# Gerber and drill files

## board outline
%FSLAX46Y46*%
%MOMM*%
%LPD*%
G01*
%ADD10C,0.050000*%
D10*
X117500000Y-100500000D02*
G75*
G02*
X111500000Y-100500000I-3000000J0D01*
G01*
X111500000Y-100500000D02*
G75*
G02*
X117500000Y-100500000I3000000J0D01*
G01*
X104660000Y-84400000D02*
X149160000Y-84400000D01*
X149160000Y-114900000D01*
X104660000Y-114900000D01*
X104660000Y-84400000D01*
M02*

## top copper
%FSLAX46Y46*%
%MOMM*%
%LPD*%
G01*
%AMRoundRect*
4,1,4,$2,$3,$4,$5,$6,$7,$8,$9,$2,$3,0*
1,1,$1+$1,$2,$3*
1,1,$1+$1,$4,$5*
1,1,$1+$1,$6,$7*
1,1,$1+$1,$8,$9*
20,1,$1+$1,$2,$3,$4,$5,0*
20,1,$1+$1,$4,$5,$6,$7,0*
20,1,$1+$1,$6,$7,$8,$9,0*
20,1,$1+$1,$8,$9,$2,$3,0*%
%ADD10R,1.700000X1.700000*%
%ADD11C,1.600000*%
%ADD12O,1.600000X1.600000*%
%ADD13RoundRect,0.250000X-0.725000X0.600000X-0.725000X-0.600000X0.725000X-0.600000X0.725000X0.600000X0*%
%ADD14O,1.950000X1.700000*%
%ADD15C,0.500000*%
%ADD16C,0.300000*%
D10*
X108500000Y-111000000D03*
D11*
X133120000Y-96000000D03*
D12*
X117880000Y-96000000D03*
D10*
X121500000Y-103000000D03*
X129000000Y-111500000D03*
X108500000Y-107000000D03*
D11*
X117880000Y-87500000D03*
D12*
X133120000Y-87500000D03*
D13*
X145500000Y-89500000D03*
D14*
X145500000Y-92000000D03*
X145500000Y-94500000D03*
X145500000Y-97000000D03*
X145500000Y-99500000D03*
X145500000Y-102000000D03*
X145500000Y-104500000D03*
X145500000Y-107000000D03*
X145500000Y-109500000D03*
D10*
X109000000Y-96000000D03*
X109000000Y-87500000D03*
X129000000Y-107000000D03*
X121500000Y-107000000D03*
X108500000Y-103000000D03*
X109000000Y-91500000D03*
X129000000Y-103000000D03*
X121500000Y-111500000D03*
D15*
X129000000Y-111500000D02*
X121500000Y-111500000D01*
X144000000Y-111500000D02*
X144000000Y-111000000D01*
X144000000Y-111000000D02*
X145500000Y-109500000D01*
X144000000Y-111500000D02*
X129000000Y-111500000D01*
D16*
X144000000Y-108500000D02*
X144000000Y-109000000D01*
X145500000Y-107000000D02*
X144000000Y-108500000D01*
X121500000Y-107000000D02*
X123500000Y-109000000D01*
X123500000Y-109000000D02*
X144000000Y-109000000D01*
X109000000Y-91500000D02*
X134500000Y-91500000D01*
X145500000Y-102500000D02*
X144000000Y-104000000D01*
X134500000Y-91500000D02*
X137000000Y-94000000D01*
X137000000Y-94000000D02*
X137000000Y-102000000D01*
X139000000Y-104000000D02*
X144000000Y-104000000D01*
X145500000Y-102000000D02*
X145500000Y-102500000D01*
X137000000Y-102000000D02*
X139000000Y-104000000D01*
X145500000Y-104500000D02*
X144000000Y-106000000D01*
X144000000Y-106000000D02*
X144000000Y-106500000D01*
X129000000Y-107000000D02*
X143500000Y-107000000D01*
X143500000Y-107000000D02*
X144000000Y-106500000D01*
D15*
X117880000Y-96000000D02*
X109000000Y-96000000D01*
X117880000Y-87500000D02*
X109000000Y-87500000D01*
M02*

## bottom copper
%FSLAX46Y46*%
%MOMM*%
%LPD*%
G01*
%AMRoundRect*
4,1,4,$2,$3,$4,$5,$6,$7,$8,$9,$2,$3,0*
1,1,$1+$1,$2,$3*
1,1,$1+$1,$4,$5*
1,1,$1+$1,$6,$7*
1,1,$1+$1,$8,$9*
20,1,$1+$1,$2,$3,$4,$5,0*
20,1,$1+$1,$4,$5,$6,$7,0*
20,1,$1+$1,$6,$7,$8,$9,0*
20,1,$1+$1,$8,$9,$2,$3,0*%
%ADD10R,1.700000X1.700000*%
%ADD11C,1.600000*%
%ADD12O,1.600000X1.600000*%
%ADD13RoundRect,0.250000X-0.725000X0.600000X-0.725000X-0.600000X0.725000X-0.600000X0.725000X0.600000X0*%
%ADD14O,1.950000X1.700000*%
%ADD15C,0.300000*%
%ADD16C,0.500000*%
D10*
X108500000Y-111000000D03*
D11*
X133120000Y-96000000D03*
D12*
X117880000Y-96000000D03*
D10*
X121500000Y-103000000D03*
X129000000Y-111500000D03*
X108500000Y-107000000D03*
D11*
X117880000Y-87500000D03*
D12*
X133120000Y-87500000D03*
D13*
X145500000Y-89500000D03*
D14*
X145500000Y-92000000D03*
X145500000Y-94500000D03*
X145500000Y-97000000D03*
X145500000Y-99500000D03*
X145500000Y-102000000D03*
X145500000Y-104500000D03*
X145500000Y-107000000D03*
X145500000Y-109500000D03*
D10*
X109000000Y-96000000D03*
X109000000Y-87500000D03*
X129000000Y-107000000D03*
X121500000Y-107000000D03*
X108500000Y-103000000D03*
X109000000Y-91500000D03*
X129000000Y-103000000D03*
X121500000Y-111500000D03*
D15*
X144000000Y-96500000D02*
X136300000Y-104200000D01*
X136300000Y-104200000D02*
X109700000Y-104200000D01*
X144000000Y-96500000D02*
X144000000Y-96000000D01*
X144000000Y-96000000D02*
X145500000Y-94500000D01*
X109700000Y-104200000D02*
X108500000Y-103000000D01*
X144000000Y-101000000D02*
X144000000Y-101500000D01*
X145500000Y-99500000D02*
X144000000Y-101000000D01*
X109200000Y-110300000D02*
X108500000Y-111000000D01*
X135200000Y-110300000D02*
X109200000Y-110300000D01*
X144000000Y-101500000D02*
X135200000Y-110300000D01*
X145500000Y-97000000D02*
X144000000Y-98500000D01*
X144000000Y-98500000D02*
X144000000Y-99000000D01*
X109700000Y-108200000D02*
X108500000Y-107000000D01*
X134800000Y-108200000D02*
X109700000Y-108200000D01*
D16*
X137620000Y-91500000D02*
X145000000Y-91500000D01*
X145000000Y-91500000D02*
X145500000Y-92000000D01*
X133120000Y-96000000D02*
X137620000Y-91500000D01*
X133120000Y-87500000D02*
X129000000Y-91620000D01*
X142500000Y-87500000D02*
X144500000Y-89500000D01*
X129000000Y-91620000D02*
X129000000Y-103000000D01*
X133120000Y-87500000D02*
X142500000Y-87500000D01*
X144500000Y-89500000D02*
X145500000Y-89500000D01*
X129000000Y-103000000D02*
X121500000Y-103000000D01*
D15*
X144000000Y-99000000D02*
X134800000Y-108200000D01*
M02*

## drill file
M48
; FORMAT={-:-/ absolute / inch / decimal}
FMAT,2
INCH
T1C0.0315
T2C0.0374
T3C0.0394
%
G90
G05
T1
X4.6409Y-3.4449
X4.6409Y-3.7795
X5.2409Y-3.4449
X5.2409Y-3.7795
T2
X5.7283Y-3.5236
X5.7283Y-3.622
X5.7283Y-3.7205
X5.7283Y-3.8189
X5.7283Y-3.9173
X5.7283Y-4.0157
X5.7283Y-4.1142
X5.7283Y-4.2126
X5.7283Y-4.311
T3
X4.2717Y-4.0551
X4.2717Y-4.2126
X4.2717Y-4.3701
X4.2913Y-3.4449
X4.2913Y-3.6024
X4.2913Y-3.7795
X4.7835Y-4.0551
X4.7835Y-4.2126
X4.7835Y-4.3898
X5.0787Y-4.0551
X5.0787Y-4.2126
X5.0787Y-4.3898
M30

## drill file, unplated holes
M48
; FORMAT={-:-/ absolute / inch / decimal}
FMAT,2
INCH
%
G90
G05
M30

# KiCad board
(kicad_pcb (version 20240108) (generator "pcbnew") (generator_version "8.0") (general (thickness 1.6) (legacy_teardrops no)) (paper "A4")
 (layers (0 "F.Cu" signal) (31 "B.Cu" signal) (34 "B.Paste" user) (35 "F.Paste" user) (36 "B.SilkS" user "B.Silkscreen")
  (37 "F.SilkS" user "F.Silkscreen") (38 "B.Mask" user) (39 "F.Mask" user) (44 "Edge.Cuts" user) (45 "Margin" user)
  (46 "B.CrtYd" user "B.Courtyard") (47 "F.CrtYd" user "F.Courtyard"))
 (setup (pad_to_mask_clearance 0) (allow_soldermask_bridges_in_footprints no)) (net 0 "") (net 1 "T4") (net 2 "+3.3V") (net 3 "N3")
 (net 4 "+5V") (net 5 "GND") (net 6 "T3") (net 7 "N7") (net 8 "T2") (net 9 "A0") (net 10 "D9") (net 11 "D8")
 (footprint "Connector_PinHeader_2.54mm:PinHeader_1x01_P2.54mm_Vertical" (layer "F.Cu") (at 108.5 111 -90)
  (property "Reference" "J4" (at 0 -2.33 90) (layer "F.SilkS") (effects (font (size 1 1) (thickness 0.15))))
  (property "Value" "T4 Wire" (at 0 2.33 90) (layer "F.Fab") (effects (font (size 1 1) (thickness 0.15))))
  (pad "1" thru_hole rect (at 0 0 270) (size 1.7 1.7) (drill 1) (layers "*.Cu" "*.Mask") (remove_unused_layers no) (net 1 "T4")))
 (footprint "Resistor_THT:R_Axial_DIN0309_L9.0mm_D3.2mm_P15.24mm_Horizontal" (layer "F.Cu") (at 133.12 96 180)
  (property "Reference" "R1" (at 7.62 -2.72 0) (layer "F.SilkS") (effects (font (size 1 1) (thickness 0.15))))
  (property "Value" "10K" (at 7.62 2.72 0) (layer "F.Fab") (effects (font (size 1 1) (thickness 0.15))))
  (pad "1" thru_hole circle (at 0 0 180) (size 1.6 1.6) (drill 0.8) (layers "*.Cu" "*.Mask") (remove_unused_layers no) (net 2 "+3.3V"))
  (pad "2" thru_hole oval (at 15.24 0 180) (size 1.6 1.6) (drill 0.8) (layers "*.Cu" "*.Mask") (remove_unused_layers no) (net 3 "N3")))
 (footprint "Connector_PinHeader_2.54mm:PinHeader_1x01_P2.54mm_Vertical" (layer "F.Cu") (at 121.5 103 -90)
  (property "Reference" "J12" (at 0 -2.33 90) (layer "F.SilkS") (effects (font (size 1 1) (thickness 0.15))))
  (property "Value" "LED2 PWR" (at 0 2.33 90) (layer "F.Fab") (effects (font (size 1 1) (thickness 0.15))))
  (pad "1" thru_hole rect (at 0 0 270) (size 1.7 1.7) (drill 1) (layers "*.Cu" "*.Mask") (remove_unused_layers no) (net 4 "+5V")))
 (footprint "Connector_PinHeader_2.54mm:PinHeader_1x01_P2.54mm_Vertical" (layer "F.Cu") (at 129 111.5 -90)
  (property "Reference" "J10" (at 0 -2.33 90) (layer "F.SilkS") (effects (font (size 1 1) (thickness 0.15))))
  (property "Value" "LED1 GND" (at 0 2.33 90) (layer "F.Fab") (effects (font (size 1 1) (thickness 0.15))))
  (pad "1" thru_hole rect (at 0 0 270) (size 1.7 1.7) (drill 1) (layers "*.Cu" "*.Mask") (remove_unused_layers no) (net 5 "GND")))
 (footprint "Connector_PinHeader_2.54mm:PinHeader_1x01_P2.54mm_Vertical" (layer "F.Cu") (at 108.5 107 -90)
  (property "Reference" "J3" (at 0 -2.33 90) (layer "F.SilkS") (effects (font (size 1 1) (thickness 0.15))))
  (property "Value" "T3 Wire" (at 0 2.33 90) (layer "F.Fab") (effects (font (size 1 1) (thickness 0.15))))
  (pad "1" thru_hole rect (at 0 0 270) (size 1.7 1.7) (drill 1) (layers "*.Cu" "*.Mask") (remove_unused_layers no) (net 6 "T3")))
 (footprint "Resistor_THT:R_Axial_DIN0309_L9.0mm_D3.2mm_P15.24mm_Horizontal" (layer "F.Cu") (at 117.88 87.5)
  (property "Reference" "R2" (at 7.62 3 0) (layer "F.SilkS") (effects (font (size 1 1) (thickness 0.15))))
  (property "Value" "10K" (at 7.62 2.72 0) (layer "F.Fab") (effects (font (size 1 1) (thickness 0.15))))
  (pad "1" thru_hole circle (at 0 0) (size 1.6 1.6) (drill 0.8) (layers "*.Cu" "*.Mask") (remove_unused_layers no) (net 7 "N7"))
  (pad "2" thru_hole oval (at 15.24 0) (size 1.6 1.6) (drill 0.8) (layers "*.Cu" "*.Mask") (remove_unused_layers no) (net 4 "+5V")))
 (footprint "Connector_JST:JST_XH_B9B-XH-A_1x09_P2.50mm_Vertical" (layer "F.Cu") (at 145.5 89.5 -90)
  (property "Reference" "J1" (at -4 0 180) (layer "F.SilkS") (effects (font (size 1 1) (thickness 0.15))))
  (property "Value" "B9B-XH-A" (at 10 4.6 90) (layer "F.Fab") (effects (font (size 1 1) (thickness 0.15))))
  (pad "1" thru_hole roundrect (at 0 0 270) (size 1.7 1.95) (drill 0.95) (layers "*.Cu" "*.Mask") (remove_unused_layers no)
   (roundrect_rratio 0.147059) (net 4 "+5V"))
  (pad "2" thru_hole oval (at 2.5 0 270) (size 1.7 1.95) (drill 0.95) (layers "*.Cu" "*.Mask") (remove_unused_layers no) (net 2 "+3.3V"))
  (pad "3" thru_hole oval (at 5 0 270) (size 1.7 1.95) (drill 0.95) (layers "*.Cu" "*.Mask") (remove_unused_layers no) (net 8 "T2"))
  (pad "4" thru_hole oval (at 7.5 0 270) (size 1.7 1.95) (drill 0.95) (layers "*.Cu" "*.Mask") (remove_unused_layers no) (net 6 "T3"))
  (pad "5" thru_hole oval (at 10 0 270) (size 1.7 1.95) (drill 0.95) (layers "*.Cu" "*.Mask") (remove_unused_layers no) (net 1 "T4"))
  (pad "6" thru_hole oval (at 12.5 0 270) (size 1.7 1.95) (drill 0.95) (layers "*.Cu" "*.Mask") (remove_unused_layers no) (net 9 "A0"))
  (pad "7" thru_hole oval (at 15 0 270) (size 1.7 1.95) (drill 0.95) (layers "*.Cu" "*.Mask") (remove_unused_layers no) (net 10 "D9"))
  (pad "8" thru_hole oval (at 17.5 0 270) (size 1.7 1.95) (drill 0.95) (layers "*.Cu" "*.Mask") (remove_unused_layers no) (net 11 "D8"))
  (pad "9" thru_hole oval (at 20 0 270) (size 1.7 1.95) (drill 0.95) (layers "*.Cu" "*.Mask") (remove_unused_layers no) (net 5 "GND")))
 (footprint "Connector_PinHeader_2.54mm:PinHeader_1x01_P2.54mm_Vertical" (layer "F.Cu") (at 109 96 -90)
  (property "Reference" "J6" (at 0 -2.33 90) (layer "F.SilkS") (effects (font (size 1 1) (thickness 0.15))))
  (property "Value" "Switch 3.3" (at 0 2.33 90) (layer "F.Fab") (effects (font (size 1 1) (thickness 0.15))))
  (pad "1" thru_hole rect (at 0 0 270) (size 1.7 1.7) (drill 1) (layers "*.Cu" "*.Mask") (remove_unused_layers no) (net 3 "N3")))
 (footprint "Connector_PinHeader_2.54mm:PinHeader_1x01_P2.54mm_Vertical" (layer "F.Cu") (at 109 87.5 -90)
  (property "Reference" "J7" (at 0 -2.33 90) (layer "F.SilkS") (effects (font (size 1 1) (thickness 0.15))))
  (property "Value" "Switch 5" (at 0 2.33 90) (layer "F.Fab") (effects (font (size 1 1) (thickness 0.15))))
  (pad "1" thru_hole rect (at 0 0 270) (size 1.7 1.7) (drill 1) (layers "*.Cu" "*.Mask") (remove_unused_layers no) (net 7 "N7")))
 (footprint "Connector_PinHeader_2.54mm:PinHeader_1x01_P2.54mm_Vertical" (layer "F.Cu") (at 129 107 -90)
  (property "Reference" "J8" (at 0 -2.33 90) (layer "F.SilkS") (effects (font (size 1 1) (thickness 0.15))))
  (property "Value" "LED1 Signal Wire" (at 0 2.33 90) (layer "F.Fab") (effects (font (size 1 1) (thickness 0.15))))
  (pad "1" thru_hole rect (at 0 0 270) (size 1.7 1.7) (drill 1) (layers "*.Cu" "*.Mask") (remove_unused_layers no) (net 10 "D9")))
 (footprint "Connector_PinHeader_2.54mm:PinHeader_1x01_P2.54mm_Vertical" (layer "F.Cu") (at 121.5 107 -90)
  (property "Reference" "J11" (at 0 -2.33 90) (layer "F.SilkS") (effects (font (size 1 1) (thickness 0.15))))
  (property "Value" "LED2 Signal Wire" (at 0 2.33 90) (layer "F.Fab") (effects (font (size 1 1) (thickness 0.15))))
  (pad "1" thru_hole rect (at 0 0 270) (size 1.7 1.7) (drill 1) (layers "*.Cu" "*.Mask") (remove_unused_layers no) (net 11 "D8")))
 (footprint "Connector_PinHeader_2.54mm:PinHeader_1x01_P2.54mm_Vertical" (layer "F.Cu") (at 108.5 103 -90)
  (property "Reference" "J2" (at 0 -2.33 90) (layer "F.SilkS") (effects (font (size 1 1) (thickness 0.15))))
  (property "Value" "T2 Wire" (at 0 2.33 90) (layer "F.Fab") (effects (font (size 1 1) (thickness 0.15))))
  (pad "1" thru_hole rect (at 0 0 270) (size 1.7 1.7) (drill 1) (layers "*.Cu" "*.Mask") (remove_unused_layers no) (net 8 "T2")))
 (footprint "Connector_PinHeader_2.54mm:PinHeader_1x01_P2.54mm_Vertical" (layer "F.Cu") (at 109 91.5 -90)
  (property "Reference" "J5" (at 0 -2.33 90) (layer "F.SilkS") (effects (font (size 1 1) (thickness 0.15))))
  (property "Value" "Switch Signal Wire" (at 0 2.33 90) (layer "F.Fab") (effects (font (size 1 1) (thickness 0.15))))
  (pad "1" thru_hole rect (at 0 0 270) (size 1.7 1.7) (drill 1) (layers "*.Cu" "*.Mask") (remove_unused_layers no) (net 9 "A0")))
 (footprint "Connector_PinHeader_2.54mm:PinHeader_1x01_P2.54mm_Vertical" (layer "F.Cu") (at 129 103 -90)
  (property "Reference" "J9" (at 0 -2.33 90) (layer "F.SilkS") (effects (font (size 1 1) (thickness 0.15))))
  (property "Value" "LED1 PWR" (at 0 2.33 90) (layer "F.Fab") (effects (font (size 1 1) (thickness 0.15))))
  (pad "1" thru_hole rect (at 0 0 270) (size 1.7 1.7) (drill 1) (layers "*.Cu" "*.Mask") (remove_unused_layers no) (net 4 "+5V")))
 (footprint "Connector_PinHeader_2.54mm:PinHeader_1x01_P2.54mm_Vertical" (layer "F.Cu") (at 121.5 111.5 -90)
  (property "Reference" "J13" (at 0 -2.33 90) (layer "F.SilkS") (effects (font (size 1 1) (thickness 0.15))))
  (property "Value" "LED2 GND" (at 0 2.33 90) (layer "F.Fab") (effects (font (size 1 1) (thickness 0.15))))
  (pad "1" thru_hole rect (at 0 0 270) (size 1.7 1.7) (drill 1) (layers "*.Cu" "*.Mask") (remove_unused_layers no) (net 5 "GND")))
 (gr_circle (center 114.5 100.5) (end 117.5 100.5) (stroke (width 0.05) (type default)) (fill none) (layer "Edge.Cuts"))
 (gr_rect (start 104.66 84.4) (end 149.16 114.9) (stroke (width 0.05) (type default)) (fill none) (layer "Edge.Cuts"))
 (segment (start 144 96.5) (end 136.3 104.2) (width 0.3) (layer "B.Cu") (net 8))
 (segment (start 136.3 104.2) (end 109.7 104.2) (width 0.3) (layer "B.Cu") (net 8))
 (segment (start 144 96.5) (end 144 96) (width 0.3) (layer "B.Cu") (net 8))
 (segment (start 144 96) (end 145.5 94.5) (width 0.3) (layer "B.Cu") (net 8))
 (segment (start 109.7 104.2) (end 108.5 103) (width 0.3) (layer "B.Cu") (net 8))
 (segment (start 129 111.5) (end 121.5 111.5) (width 0.5) (layer "F.Cu") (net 5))
 (segment (start 144 111.5) (end 144 111) (width 0.5) (layer "F.Cu") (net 5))
 (segment (start 144 111) (end 145.5 109.5) (width 0.5) (layer "F.Cu") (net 5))
 (segment (start 144 111.5) (end 129 111.5) (width 0.5) (layer "F.Cu") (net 5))
 (segment (start 144 108.5) (end 144 109) (width 0.3) (layer "F.Cu") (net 11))
 (segment (start 145.5 107) (end 144 108.5) (width 0.3) (layer "F.Cu") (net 11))
 (segment (start 121.5 107) (end 123.5 109) (width 0.3) (layer "F.Cu") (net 11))
 (segment (start 123.5 109) (end 144 109) (width 0.3) (layer "F.Cu") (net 11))
 (segment (start 144 101) (end 144 101.5) (width 0.3) (layer "B.Cu") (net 1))
 (segment (start 145.5 99.5) (end 144 101) (width 0.3) (layer "B.Cu") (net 1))
 (segment (start 109.2 110.3) (end 108.5 111) (width 0.3) (layer "B.Cu") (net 1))
 (segment (start 135.2 110.3) (end 109.2 110.3) (width 0.3) (layer "B.Cu") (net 1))
 (segment (start 144 101.5) (end 135.2 110.3) (width 0.3) (layer "B.Cu") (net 1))
 (segment (start 109 91.5) (end 134.5 91.5) (width 0.3) (layer "F.Cu") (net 9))
 (segment (start 145.5 102.5) (end 144 104) (width 0.3) (layer "F.Cu") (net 9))
 (segment (start 134.5 91.5) (end 137 94) (width 0.3) (layer "F.Cu") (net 9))
 (segment (start 137 94) (end 137 102) (width 0.3) (layer "F.Cu") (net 9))
 (segment (start 139 104) (end 144 104) (width 0.3) (layer "F.Cu") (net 9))
 (segment (start 145.5 102) (end 145.5 102.5) (width 0.3) (layer "F.Cu") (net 9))
 (segment (start 137 102) (end 139 104) (width 0.3) (layer "F.Cu") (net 9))
 (segment (start 145.5 97) (end 144 98.5) (width 0.3) (layer "B.Cu") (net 6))
 (segment (start 144 99) (end 134.8 108.2) (width 0.3) (layer "B.Cu") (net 6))
 (segment (start 144 98.5) (end 144 99) (width 0.3) (layer "B.Cu") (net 6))
 (segment (start 109.7 108.2) (end 108.5 107) (width 0.3) (layer "B.Cu") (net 6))
 (segment (start 134.8 108.2) (end 109.7 108.2) (width 0.3) (layer "B.Cu") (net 6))
 (segment (start 137.62 91.5) (end 145 91.5) (width 0.5) (layer "B.Cu") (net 2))
 (segment (start 145 91.5) (end 145.5 92) (width 0.5) (layer "B.Cu") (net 2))
 (segment (start 133.12 96) (end 137.62 91.5) (width 0.5) (layer "B.Cu") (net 2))
 (segment (start 145.5 104.5) (end 144 106) (width 0.3) (layer "F.Cu") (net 10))
 (segment (start 144 106) (end 144 106.5) (width 0.3) (layer "F.Cu") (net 10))
 (segment (start 129 107) (end 143.5 107) (width 0.3) (layer "F.Cu") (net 10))
 (segment (start 143.5 107) (end 144 106.5) (width 0.3) (layer "F.Cu") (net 10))
 (segment (start 117.88 96) (end 109 96) (width 0.5) (layer "F.Cu") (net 3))
 (segment (start 117.88 87.5) (end 109 87.5) (width 0.5) (layer "F.Cu") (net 7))
 (segment (start 133.12 87.5) (end 129 91.62) (width 0.5) (layer "B.Cu") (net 4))
 (segment (start 142.5 87.5) (end 144.5 89.5) (width 0.5) (layer "B.Cu") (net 4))
 (segment (start 129 91.62) (end 129 103) (width 0.5) (layer "B.Cu") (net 4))
 (segment (start 133.12 87.5) (end 142.5 87.5) (width 0.5) (layer "B.Cu") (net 4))
 (segment (start 144.5 89.5) (end 145.5 89.5) (width 0.5) (layer "B.Cu") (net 4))
 (segment (start 129 103) (end 121.5 103) (width 0.5) (layer "B.Cu") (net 4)))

